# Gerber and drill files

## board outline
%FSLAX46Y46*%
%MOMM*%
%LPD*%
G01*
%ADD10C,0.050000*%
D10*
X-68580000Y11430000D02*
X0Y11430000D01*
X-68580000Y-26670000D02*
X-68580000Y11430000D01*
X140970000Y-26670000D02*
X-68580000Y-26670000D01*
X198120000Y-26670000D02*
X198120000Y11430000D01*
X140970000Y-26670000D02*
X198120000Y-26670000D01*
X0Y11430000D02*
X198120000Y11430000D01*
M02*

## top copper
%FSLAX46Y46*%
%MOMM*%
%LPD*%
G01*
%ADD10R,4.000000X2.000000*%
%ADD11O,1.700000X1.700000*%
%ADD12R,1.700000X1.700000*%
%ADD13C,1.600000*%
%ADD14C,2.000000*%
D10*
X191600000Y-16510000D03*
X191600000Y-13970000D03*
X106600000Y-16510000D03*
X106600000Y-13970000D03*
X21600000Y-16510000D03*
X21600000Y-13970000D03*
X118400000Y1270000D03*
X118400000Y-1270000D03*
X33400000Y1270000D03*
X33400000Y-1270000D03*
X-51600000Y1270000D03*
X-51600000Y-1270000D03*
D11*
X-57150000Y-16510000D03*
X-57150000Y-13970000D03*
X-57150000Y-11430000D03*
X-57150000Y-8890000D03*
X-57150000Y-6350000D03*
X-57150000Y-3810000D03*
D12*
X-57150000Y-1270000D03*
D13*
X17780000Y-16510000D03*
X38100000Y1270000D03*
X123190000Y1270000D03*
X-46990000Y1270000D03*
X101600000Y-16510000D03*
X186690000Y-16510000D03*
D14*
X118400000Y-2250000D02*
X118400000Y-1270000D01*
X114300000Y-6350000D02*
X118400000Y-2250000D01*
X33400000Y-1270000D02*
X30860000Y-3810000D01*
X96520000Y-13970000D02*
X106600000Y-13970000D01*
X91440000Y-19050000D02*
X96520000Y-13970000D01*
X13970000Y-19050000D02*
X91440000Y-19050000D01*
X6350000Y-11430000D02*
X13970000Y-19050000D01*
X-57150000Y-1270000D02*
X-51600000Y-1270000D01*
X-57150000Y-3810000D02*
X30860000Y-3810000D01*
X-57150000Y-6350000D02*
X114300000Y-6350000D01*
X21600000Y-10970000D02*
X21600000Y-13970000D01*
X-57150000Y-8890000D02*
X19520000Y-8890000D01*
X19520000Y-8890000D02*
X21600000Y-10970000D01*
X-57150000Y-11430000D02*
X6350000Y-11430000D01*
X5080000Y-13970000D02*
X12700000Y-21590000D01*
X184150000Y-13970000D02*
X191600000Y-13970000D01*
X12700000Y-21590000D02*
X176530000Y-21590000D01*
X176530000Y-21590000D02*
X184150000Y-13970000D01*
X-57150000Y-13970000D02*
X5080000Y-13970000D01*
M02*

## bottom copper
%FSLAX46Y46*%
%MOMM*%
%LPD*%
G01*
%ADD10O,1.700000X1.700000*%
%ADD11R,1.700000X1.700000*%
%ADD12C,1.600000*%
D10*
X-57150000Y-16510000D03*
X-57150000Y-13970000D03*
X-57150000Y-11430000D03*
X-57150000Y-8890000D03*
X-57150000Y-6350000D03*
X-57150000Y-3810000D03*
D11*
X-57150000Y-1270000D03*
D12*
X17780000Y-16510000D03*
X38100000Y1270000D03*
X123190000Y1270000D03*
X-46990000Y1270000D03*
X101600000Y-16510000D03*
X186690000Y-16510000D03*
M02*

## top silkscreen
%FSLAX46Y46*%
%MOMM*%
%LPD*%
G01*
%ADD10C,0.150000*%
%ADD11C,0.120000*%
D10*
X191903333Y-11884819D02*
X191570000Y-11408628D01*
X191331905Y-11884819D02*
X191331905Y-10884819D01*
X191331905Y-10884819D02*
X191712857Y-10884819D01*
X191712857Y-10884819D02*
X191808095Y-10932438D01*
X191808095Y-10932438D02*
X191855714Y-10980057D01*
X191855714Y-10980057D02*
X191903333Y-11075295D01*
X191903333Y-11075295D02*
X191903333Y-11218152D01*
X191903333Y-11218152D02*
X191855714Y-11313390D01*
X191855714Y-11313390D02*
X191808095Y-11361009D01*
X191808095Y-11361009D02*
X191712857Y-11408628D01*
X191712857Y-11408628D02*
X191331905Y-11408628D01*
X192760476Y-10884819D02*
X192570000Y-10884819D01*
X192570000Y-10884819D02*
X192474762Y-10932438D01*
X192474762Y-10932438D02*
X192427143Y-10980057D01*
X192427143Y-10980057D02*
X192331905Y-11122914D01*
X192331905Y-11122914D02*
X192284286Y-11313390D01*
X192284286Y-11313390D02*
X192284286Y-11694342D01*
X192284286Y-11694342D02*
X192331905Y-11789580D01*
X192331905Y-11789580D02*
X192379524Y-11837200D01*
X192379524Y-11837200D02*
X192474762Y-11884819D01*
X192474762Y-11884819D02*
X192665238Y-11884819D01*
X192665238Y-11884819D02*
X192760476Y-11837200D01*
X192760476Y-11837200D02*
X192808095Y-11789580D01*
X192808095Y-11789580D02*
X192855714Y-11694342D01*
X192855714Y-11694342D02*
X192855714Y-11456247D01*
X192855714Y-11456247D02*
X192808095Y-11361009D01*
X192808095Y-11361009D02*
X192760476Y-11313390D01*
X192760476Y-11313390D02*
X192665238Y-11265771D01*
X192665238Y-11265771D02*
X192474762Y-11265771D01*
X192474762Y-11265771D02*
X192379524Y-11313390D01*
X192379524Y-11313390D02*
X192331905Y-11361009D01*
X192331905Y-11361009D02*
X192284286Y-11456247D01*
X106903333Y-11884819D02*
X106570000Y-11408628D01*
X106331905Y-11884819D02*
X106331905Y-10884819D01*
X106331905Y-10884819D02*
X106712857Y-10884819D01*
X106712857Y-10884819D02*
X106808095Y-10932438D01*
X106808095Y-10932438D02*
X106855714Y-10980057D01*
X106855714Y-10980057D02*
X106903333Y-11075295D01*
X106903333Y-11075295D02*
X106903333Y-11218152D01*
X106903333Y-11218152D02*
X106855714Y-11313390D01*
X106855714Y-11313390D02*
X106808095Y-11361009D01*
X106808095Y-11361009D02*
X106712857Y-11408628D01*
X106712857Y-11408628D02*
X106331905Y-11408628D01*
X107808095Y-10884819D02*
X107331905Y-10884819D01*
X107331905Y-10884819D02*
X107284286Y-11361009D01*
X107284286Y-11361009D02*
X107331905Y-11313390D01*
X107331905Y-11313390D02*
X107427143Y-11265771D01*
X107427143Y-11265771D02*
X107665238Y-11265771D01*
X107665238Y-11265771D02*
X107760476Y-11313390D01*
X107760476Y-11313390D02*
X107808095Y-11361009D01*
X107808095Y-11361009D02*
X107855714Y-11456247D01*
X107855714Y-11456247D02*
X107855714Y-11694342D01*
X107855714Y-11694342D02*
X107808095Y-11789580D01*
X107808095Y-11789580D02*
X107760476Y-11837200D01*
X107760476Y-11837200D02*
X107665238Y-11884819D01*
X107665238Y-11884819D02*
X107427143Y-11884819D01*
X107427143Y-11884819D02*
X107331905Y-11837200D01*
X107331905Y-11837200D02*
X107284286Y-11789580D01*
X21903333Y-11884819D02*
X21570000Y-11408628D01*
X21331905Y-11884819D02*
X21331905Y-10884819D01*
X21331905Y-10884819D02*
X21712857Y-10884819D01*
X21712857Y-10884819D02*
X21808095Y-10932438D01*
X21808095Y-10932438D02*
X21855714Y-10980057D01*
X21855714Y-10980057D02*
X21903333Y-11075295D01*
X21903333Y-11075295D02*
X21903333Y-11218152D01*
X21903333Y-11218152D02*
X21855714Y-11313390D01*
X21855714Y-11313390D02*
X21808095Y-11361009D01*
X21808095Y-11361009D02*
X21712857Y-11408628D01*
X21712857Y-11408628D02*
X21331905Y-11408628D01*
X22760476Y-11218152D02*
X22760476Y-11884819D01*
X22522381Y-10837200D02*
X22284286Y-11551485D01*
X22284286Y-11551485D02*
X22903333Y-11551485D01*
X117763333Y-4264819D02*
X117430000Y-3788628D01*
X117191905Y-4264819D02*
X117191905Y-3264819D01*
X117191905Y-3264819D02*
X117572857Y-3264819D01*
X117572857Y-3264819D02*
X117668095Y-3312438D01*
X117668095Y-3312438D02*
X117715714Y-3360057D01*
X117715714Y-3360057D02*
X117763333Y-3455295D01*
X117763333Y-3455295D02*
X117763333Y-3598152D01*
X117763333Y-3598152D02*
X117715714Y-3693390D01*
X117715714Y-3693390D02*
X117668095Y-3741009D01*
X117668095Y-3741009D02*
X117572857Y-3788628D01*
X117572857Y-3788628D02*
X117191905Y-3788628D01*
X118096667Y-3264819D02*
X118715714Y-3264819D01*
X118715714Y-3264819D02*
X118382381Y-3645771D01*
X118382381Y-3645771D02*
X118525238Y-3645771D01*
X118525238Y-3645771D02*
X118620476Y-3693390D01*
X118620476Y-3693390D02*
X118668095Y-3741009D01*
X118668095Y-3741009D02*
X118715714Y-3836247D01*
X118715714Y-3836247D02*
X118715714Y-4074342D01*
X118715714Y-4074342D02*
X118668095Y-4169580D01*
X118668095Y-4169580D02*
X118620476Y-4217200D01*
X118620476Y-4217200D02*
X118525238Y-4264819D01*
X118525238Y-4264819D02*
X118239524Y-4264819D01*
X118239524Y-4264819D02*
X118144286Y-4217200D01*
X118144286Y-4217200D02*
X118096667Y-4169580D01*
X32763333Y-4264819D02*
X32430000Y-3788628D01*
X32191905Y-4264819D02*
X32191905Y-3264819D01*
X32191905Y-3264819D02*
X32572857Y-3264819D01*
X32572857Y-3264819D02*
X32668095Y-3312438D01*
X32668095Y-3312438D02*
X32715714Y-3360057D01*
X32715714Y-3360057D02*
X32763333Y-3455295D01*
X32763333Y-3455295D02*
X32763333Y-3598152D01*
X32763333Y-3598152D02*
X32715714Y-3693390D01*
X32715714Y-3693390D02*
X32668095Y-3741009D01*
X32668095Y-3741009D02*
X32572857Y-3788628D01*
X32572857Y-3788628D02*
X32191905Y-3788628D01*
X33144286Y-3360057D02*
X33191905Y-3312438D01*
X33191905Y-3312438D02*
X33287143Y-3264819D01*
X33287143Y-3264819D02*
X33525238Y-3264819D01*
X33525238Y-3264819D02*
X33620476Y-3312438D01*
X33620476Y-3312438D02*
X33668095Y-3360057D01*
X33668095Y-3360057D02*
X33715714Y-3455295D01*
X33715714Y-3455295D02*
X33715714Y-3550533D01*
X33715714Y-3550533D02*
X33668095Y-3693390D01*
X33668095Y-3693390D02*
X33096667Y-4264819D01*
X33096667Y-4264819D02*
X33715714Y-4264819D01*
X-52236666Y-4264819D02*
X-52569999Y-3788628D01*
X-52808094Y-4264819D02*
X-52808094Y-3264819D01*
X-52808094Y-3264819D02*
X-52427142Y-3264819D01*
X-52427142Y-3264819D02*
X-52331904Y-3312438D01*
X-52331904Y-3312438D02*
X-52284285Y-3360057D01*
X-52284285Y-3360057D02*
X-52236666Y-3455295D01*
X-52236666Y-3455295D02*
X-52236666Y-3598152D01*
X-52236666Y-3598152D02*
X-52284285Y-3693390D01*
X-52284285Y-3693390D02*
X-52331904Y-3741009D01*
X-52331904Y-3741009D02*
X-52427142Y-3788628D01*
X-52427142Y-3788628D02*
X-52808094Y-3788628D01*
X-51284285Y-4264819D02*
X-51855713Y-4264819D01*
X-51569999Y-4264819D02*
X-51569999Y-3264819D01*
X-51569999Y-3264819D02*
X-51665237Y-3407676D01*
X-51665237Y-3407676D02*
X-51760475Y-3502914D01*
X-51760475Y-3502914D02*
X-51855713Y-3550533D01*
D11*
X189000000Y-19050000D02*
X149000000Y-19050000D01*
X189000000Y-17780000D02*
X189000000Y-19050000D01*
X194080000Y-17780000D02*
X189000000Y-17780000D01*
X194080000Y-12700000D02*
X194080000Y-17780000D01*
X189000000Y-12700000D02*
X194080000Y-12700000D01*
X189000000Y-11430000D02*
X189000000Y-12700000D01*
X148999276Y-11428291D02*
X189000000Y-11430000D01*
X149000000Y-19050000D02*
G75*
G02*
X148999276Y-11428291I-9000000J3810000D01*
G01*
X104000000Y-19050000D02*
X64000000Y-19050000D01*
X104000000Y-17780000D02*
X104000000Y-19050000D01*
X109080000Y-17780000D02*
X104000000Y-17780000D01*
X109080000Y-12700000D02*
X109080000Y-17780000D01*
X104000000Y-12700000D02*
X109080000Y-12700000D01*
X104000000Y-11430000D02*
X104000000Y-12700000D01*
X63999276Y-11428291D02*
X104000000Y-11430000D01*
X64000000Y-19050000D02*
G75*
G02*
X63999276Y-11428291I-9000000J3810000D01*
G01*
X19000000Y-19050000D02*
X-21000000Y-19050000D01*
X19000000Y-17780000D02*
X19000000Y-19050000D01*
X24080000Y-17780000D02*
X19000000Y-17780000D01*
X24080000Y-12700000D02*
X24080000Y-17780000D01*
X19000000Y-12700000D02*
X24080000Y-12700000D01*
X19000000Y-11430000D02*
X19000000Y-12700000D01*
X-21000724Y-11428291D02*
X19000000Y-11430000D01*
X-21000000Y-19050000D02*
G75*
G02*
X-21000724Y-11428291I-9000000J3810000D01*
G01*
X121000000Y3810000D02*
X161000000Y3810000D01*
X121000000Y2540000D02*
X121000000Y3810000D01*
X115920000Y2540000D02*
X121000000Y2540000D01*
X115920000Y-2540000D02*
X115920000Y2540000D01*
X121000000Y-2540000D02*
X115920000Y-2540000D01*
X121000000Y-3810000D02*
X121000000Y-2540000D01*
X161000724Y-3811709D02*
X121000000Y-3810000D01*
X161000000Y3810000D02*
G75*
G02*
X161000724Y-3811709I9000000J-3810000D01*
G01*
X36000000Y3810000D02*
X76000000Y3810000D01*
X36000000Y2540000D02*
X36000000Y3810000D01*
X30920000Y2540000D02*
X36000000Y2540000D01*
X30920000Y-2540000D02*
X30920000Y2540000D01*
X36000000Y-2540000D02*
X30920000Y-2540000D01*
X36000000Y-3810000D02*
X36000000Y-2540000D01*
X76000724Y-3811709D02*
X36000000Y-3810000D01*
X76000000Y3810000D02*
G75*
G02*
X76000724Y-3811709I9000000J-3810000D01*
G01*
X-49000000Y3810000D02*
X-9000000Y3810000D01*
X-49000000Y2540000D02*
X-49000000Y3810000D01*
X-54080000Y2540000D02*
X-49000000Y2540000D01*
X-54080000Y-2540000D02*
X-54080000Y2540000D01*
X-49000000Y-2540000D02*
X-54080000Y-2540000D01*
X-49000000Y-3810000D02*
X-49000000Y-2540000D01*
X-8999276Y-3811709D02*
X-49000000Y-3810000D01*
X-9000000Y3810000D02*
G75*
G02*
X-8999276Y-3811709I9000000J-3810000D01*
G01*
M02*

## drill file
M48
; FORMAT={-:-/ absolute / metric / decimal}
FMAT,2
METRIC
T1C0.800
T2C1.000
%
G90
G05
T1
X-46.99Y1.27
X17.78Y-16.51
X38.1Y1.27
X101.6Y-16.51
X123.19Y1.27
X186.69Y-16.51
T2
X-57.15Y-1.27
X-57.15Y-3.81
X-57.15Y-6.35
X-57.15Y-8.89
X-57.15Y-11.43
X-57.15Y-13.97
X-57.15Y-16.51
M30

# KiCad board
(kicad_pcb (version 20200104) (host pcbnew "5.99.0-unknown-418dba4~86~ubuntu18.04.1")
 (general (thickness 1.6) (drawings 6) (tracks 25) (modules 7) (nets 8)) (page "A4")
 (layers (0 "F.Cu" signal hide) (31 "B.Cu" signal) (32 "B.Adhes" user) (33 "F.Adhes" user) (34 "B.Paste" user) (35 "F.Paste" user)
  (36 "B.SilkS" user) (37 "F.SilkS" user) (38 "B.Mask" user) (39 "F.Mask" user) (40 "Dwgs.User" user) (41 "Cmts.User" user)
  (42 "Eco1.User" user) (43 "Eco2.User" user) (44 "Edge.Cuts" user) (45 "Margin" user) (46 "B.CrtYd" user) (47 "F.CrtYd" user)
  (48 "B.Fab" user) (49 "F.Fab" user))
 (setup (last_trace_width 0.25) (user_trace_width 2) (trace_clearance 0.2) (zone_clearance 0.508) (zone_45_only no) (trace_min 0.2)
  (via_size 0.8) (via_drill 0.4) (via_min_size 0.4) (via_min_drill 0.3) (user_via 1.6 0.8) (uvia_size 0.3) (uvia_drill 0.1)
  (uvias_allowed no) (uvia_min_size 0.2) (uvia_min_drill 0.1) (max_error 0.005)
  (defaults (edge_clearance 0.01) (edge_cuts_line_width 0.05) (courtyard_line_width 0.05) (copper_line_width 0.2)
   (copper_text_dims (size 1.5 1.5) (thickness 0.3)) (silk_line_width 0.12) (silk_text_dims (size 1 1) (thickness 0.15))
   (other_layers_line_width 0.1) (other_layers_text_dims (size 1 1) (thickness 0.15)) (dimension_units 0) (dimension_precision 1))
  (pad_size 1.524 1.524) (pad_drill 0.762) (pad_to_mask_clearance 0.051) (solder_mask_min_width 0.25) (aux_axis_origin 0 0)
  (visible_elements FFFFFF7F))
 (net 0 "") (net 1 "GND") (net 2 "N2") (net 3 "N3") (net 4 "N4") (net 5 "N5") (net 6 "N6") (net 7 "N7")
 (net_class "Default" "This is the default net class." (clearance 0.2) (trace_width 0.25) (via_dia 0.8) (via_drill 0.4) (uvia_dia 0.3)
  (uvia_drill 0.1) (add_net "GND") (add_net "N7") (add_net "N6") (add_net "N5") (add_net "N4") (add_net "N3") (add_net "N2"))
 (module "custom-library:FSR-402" (layer "F.Cu") (at 140 15.24)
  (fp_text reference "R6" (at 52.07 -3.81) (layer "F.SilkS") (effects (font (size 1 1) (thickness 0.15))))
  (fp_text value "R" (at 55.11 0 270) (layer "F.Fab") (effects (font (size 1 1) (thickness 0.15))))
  (fp_line (start 49 3.81) (end 9 3.81) (layer "F.SilkS") (width 0.12))
  (fp_line (start 49 2.54) (end 49 3.81) (layer "F.SilkS") (width 0.12))
  (fp_line (start 54.08 2.54) (end 49 2.54) (layer "F.SilkS") (width 0.12))
  (fp_line (start 54.08 -2.54) (end 54.08 2.54) (layer "F.SilkS") (width 0.12))
  (fp_line (start 49 -2.54) (end 54.08 -2.54) (layer "F.SilkS") (width 0.12))
  (fp_line (start 49 -3.81) (end 49 -2.54) (layer "F.SilkS") (width 0.12))
  (fp_line (start 8.999276 -3.811709) (end 49 -3.81) (layer "F.SilkS") (width 0.12))
  (fp_arc (start 0 0) (end 9 3.81) (angle 314.1) (layer "F.SilkS") (width 0.12))
  (pad "2" smd rect (at 51.6 1.27 270) (size 2 4) (layers "F.Cu" "F.Paste" "F.Mask") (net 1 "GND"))
  (pad "1" smd rect (at 51.6 -1.27 270) (size 2 4) (layers "F.Cu" "F.Paste" "F.Mask") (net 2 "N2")))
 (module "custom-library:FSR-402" (layer "F.Cu") (at 55 15.24)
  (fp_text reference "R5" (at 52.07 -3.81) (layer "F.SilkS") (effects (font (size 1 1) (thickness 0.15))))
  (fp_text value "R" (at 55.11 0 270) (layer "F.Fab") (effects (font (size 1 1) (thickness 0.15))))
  (fp_line (start 49 3.81) (end 9 3.81) (layer "F.SilkS") (width 0.12))
  (fp_line (start 49 2.54) (end 49 3.81) (layer "F.SilkS") (width 0.12))
  (fp_line (start 54.08 2.54) (end 49 2.54) (layer "F.SilkS") (width 0.12))
  (fp_line (start 54.08 -2.54) (end 54.08 2.54) (layer "F.SilkS") (width 0.12))
  (fp_line (start 49 -2.54) (end 54.08 -2.54) (layer "F.SilkS") (width 0.12))
  (fp_line (start 49 -3.81) (end 49 -2.54) (layer "F.SilkS") (width 0.12))
  (fp_line (start 8.999276 -3.811709) (end 49 -3.81) (layer "F.SilkS") (width 0.12))
  (fp_arc (start 0 0) (end 9 3.81) (angle 314.1) (layer "F.SilkS") (width 0.12))
  (pad "2" smd rect (at 51.6 1.27 270) (size 2 4) (layers "F.Cu" "F.Paste" "F.Mask") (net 1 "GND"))
  (pad "1" smd rect (at 51.6 -1.27 270) (size 2 4) (layers "F.Cu" "F.Paste" "F.Mask") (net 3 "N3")))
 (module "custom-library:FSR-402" (layer "F.Cu") (at -30 15.24)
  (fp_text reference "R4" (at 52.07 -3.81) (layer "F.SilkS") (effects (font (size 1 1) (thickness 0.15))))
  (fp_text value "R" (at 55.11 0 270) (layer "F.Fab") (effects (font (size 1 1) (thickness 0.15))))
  (fp_line (start 49 3.81) (end 9 3.81) (layer "F.SilkS") (width 0.12))
  (fp_line (start 49 2.54) (end 49 3.81) (layer "F.SilkS") (width 0.12))
  (fp_line (start 54.08 2.54) (end 49 2.54) (layer "F.SilkS") (width 0.12))
  (fp_line (start 54.08 -2.54) (end 54.08 2.54) (layer "F.SilkS") (width 0.12))
  (fp_line (start 49 -2.54) (end 54.08 -2.54) (layer "F.SilkS") (width 0.12))
  (fp_line (start 49 -3.81) (end 49 -2.54) (layer "F.SilkS") (width 0.12))
  (fp_line (start 8.999276 -3.811709) (end 49 -3.81) (layer "F.SilkS") (width 0.12))
  (fp_arc (start 0 0) (end 9 3.81) (angle 314.1) (layer "F.SilkS") (width 0.12))
  (pad "2" smd rect (at 51.6 1.27 270) (size 2 4) (layers "F.Cu" "F.Paste" "F.Mask") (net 1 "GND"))
  (pad "1" smd rect (at 51.6 -1.27 270) (size 2 4) (layers "F.Cu" "F.Paste" "F.Mask") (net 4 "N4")))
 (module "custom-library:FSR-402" (layer "F.Cu") (at 170 0 180)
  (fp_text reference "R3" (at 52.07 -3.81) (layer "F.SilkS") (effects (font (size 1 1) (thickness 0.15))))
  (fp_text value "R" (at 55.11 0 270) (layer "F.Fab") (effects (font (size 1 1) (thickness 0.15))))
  (fp_line (start 49 3.81) (end 9 3.81) (layer "F.SilkS") (width 0.12))
  (fp_line (start 49 2.54) (end 49 3.81) (layer "F.SilkS") (width 0.12))
  (fp_line (start 54.08 2.54) (end 49 2.54) (layer "F.SilkS") (width 0.12))
  (fp_line (start 54.08 -2.54) (end 54.08 2.54) (layer "F.SilkS") (width 0.12))
  (fp_line (start 49 -2.54) (end 54.08 -2.54) (layer "F.SilkS") (width 0.12))
  (fp_line (start 49 -3.81) (end 49 -2.54) (layer "F.SilkS") (width 0.12))
  (fp_line (start 8.999276 -3.811709) (end 49 -3.81) (layer "F.SilkS") (width 0.12))
  (fp_arc (start 0 0) (end 9 3.81) (angle 314.1) (layer "F.SilkS") (width 0.12))
  (pad "2" smd rect (at 51.6 1.27 90) (size 2 4) (layers "F.Cu" "F.Paste" "F.Mask") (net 1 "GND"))
  (pad "1" smd rect (at 51.6 -1.27 90) (size 2 4) (layers "F.Cu" "F.Paste" "F.Mask") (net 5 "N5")))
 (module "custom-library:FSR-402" (layer "F.Cu") (at 85 0 180)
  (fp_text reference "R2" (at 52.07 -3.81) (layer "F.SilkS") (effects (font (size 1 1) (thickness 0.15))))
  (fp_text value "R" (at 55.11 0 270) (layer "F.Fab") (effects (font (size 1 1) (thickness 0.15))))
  (fp_line (start 49 3.81) (end 9 3.81) (layer "F.SilkS") (width 0.12))
  (fp_line (start 49 2.54) (end 49 3.81) (layer "F.SilkS") (width 0.12))
  (fp_line (start 54.08 2.54) (end 49 2.54) (layer "F.SilkS") (width 0.12))
  (fp_line (start 54.08 -2.54) (end 54.08 2.54) (layer "F.SilkS") (width 0.12))
  (fp_line (start 49 -2.54) (end 54.08 -2.54) (layer "F.SilkS") (width 0.12))
  (fp_line (start 49 -3.81) (end 49 -2.54) (layer "F.SilkS") (width 0.12))
  (fp_line (start 8.999276 -3.811709) (end 49 -3.81) (layer "F.SilkS") (width 0.12))
  (fp_arc (start 0 0) (end 9 3.81) (angle 314.1) (layer "F.SilkS") (width 0.12))
  (pad "2" smd rect (at 51.6 1.27 90) (size 2 4) (layers "F.Cu" "F.Paste" "F.Mask") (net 1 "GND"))
  (pad "1" smd rect (at 51.6 -1.27 90) (size 2 4) (layers "F.Cu" "F.Paste" "F.Mask") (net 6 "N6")))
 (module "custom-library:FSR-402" (layer "F.Cu") (at 0 0 180)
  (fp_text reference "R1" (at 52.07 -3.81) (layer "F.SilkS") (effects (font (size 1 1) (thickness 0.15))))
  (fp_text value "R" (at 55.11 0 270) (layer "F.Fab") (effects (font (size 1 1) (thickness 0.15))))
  (fp_line (start 49 3.81) (end 9 3.81) (layer "F.SilkS") (width 0.12))
  (fp_line (start 49 2.54) (end 49 3.81) (layer "F.SilkS") (width 0.12))
  (fp_line (start 54.08 2.54) (end 49 2.54) (layer "F.SilkS") (width 0.12))
  (fp_line (start 54.08 -2.54) (end 54.08 2.54) (layer "F.SilkS") (width 0.12))
  (fp_line (start 49 -2.54) (end 54.08 -2.54) (layer "F.SilkS") (width 0.12))
  (fp_line (start 49 -3.81) (end 49 -2.54) (layer "F.SilkS") (width 0.12))
  (fp_line (start 8.999276 -3.811709) (end 49 -3.81) (layer "F.SilkS") (width 0.12))
  (fp_arc (start 0 0) (end 9 3.81) (angle 314.1) (layer "F.SilkS") (width 0.12))
  (pad "2" smd rect (at 51.6 1.27 90) (size 2 4) (layers "F.Cu" "F.Paste" "F.Mask") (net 1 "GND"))
  (pad "1" smd rect (at 51.6 -1.27 90) (size 2 4) (layers "F.Cu" "F.Paste" "F.Mask") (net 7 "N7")))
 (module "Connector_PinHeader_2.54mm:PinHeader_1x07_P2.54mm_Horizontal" (layer "B.Cu") (at -57.15 1.27 180)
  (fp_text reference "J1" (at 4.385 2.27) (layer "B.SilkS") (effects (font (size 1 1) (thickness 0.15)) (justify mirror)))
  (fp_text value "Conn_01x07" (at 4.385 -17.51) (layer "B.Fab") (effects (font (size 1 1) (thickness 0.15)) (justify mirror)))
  (pad "7" thru_hole oval (at 0 -15.24 180) (size 1.7 1.7) (drill 1) (layers *.Cu *.Mask) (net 1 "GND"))
  (pad "6" thru_hole oval (at 0 -12.7 180) (size 1.7 1.7) (drill 1) (layers *.Cu *.Mask) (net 2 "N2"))
  (pad "5" thru_hole oval (at 0 -10.16 180) (size 1.7 1.7) (drill 1) (layers *.Cu *.Mask) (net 3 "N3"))
  (pad "4" thru_hole oval (at 0 -7.62 180) (size 1.7 1.7) (drill 1) (layers *.Cu *.Mask) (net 4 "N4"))
  (pad "3" thru_hole oval (at 0 -5.08 180) (size 1.7 1.7) (drill 1) (layers *.Cu *.Mask) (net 5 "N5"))
  (pad "2" thru_hole oval (at 0 -2.54 180) (size 1.7 1.7) (drill 1) (layers *.Cu *.Mask) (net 6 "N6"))
  (pad "1" thru_hole rect (at 0 0 180) (size 1.7 1.7) (drill 1) (layers *.Cu *.Mask) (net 7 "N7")))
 (gr_line (start -68.58 -11.43) (end 0 -11.43) (layer "Edge.Cuts") (width 0.05))
 (gr_line (start -68.58 26.67) (end -68.58 -11.43) (layer "Edge.Cuts") (width 0.05))
 (gr_line (start 140.97 26.67) (end -68.58 26.67) (layer "Edge.Cuts") (width 0.05))
 (gr_line (start 198.12 26.67) (end 198.12 -11.43) (layer "Edge.Cuts") (width 0.05))
 (gr_line (start 140.97 26.67) (end 198.12 26.67) (layer "Edge.Cuts") (width 0.05))
 (gr_line (start 0 -11.43) (end 198.12 -11.43) (layer "Edge.Cuts") (width 0.05))
 (segment (start 118.4 2.25) (end 118.4 1.27) (width 2) (layer "F.Cu") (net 5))
 (segment (start 114.3 6.35) (end 118.4 2.25) (width 2) (layer "F.Cu") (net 5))
 (segment (start 33.4 1.27) (end 30.86 3.81) (width 2) (layer "F.Cu") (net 6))
 (via (at 17.78 16.51) (size 1.6) (drill 0.8) (layers "F.Cu" "B.Cu") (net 1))
 (via (at 38.1 -1.27) (size 1.6) (drill 0.8) (layers "F.Cu" "B.Cu") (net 1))
 (via (at 123.19 -1.27) (size 1.6) (drill 0.8) (layers "F.Cu" "B.Cu") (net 1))
 (via (at -46.99 -1.27) (size 1.6) (drill 0.8) (layers "F.Cu" "B.Cu") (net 1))
 (via (at 101.6 16.51) (size 1.6) (drill 0.8) (layers "F.Cu" "B.Cu") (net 1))
 (via (at 186.69 16.51) (size 1.6) (drill 0.8) (layers "F.Cu" "B.Cu") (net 1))
 (segment (start 96.52 13.97) (end 106.6 13.97) (width 2) (layer "F.Cu") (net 3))
 (segment (start 91.44 19.05) (end 96.52 13.97) (width 2) (layer "F.Cu") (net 3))
 (segment (start 13.97 19.05) (end 91.44 19.05) (width 2) (layer "F.Cu") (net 3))
 (segment (start 6.35 11.43) (end 13.97 19.05) (width 2) (layer "F.Cu") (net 3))
 (segment (start -57.15 1.27) (end -51.6 1.27) (width 2) (layer "F.Cu") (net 7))
 (segment (start -57.15 3.81) (end 30.86 3.81) (width 2) (layer "F.Cu") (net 6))
 (segment (start -57.15 6.35) (end 114.3 6.35) (width 2) (layer "F.Cu") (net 5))
 (segment (start 21.6 10.97) (end 21.6 13.97) (width 2) (layer "F.Cu") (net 4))
 (segment (start -57.15 8.89) (end 19.52 8.89) (width 2) (layer "F.Cu") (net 4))
 (segment (start 19.52 8.89) (end 21.6 10.97) (width 2) (layer "F.Cu") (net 4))
 (segment (start -57.15 11.43) (end 6.35 11.43) (width 2) (layer "F.Cu") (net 3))
 (segment (start 5.08 13.97) (end 12.7 21.59) (width 2) (layer "F.Cu") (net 2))
 (segment (start 184.15 13.97) (end 191.6 13.97) (width 2) (layer "F.Cu") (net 2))
 (segment (start 12.7 21.59) (end 176.53 21.59) (width 2) (layer "F.Cu") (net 2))
 (segment (start 176.53 21.59) (end 184.15 13.97) (width 2) (layer "F.Cu") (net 2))
 (segment (start -57.15 13.97) (end 5.08 13.97) (width 2) (layer "F.Cu") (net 2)))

